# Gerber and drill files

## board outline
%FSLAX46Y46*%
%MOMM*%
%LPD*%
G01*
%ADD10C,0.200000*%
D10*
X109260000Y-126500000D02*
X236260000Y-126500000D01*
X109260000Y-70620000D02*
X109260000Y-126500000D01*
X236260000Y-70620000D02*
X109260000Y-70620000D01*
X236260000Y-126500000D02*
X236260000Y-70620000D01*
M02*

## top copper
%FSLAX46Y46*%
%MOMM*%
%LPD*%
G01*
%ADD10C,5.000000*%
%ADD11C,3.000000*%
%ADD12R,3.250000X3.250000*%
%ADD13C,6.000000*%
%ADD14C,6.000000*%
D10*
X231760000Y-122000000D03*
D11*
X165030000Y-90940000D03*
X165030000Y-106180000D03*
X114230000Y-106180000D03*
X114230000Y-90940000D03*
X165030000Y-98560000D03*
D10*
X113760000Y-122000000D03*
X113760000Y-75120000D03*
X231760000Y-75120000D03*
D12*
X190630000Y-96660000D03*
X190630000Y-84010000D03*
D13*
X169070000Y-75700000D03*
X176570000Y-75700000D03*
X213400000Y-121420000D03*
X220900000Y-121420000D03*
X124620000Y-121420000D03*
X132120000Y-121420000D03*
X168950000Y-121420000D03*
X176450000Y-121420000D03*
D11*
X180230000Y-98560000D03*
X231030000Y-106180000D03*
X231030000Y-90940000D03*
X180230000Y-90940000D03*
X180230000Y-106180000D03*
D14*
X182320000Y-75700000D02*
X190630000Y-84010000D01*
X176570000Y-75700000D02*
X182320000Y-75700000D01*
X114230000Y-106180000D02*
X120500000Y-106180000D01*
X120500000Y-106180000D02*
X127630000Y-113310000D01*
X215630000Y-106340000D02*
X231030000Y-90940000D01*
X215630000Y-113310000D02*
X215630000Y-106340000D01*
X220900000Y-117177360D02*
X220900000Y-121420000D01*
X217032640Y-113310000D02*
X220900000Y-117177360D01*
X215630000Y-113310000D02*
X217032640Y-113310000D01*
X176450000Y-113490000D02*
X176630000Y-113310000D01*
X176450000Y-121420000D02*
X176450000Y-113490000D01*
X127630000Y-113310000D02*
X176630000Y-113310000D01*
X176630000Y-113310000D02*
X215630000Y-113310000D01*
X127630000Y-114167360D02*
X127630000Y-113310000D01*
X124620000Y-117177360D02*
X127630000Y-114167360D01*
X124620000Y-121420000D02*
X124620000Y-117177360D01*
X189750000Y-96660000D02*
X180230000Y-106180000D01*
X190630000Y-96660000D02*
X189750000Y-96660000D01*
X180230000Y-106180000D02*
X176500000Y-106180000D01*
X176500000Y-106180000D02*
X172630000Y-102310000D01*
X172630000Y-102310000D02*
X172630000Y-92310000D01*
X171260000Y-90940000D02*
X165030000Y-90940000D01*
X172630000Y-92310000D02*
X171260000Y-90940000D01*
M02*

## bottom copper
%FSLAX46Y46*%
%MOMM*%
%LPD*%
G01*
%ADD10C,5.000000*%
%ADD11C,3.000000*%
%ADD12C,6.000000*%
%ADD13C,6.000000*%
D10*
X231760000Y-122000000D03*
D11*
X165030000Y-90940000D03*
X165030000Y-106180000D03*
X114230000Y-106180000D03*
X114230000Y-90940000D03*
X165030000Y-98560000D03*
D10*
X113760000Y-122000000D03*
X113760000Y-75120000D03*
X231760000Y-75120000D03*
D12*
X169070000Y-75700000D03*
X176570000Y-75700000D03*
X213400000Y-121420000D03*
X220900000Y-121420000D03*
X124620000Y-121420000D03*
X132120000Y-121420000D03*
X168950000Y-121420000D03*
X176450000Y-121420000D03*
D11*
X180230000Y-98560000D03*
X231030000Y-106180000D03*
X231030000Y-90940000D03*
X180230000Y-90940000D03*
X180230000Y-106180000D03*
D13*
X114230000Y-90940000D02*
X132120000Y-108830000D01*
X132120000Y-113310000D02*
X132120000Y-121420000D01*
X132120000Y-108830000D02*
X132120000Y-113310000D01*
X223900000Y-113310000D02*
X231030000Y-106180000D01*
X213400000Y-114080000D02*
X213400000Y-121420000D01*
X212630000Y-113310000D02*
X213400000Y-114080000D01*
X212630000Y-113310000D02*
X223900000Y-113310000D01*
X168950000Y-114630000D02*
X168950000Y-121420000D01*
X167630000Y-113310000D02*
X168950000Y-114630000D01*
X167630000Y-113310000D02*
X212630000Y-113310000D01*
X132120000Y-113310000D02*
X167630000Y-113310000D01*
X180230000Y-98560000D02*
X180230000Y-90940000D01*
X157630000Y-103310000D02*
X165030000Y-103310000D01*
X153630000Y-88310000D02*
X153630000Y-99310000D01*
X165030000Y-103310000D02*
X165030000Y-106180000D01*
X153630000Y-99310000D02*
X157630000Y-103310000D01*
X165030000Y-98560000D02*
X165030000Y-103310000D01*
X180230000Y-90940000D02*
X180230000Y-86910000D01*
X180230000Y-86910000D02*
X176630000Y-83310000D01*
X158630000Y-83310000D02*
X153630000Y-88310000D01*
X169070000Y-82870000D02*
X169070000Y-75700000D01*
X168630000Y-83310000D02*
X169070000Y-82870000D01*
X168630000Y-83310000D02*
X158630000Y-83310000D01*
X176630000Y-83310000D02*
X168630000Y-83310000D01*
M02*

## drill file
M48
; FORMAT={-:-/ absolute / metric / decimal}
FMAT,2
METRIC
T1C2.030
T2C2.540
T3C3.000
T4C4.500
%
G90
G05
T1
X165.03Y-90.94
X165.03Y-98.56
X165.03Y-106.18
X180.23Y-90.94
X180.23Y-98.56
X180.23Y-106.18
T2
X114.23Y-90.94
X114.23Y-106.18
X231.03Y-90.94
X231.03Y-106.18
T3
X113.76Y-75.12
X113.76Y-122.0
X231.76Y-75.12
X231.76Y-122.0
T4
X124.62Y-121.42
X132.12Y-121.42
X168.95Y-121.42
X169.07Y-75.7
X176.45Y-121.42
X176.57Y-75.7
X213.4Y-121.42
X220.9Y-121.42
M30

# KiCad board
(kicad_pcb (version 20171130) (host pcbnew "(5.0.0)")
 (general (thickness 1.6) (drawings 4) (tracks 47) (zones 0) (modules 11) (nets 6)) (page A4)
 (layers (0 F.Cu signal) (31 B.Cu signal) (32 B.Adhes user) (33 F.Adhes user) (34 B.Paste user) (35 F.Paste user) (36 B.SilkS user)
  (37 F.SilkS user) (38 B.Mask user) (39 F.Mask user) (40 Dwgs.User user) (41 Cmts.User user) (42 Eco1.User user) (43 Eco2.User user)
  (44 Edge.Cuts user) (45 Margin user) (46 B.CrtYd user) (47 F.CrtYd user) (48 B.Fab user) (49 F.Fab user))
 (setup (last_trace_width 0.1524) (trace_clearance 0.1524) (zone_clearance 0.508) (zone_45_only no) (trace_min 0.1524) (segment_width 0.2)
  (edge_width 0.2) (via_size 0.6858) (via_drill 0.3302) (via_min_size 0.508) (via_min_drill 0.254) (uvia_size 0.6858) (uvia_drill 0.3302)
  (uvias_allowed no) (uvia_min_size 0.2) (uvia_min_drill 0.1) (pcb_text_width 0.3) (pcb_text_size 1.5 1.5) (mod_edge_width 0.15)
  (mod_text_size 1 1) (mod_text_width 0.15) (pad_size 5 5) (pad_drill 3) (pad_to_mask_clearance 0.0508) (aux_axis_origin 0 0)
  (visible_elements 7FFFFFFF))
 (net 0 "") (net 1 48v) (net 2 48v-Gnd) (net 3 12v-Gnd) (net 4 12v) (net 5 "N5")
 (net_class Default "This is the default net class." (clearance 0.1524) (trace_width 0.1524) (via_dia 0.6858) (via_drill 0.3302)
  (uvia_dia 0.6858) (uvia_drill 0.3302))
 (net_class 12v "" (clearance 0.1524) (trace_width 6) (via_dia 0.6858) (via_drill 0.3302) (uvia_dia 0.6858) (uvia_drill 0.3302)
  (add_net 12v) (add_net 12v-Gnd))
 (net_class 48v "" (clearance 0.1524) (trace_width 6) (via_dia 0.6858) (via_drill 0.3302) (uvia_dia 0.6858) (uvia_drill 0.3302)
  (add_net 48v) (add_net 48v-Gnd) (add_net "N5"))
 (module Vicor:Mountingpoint (layer F.Cu) (at 252.73 96.52)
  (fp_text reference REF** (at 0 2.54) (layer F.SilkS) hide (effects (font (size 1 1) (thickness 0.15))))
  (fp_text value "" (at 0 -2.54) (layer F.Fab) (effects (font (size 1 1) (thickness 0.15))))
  (pad "" thru_hole circle (at -20.97 25.48) (size 5 5) (drill 3) (layers *.Cu *.Mask)))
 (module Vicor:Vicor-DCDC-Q (layer B.Cu) (at 139.63 98.56 180)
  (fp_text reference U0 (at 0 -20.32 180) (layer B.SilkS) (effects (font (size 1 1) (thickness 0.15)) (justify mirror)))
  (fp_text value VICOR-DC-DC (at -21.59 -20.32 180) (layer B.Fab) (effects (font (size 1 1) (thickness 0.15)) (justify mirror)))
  (pad 1 thru_hole circle (at -25.4 7.62 180) (size 3 3) (drill 2.03) (layers *.Cu *.Mask) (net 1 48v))
  (pad 3 thru_hole circle (at -25.4 -7.62 180) (size 3 3) (drill 2.03) (layers *.Cu *.Mask) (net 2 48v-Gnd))
  (pad 4 thru_hole circle (at 25.4 -7.62 180) (size 3 3) (drill 2.54) (layers *.Cu *.Mask) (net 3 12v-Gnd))
  (pad 5 thru_hole circle (at 25.4 7.62 180) (size 3 3) (drill 2.54) (layers *.Cu *.Mask) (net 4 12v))
  (pad 2 thru_hole circle (at -25.4 0 180) (size 3 3) (drill 2.03) (layers *.Cu *.Mask) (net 2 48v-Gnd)))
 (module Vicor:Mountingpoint (layer F.Cu) (at 263.47 99.06)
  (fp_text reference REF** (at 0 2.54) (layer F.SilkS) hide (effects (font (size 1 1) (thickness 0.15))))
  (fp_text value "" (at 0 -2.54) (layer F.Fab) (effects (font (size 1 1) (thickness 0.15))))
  (pad "" thru_hole circle (at -149.71 22.94) (size 5 5) (drill 3) (layers *.Cu *.Mask)))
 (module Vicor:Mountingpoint (layer F.Cu) (at 255.27 81.28)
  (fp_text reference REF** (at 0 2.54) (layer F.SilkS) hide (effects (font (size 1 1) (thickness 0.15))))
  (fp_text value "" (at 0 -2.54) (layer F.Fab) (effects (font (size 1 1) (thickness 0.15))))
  (pad "" thru_hole circle (at -141.51 -6.16) (size 5 5) (drill 3) (layers *.Cu *.Mask)))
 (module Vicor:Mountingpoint (layer F.Cu) (at 243.42 75.58)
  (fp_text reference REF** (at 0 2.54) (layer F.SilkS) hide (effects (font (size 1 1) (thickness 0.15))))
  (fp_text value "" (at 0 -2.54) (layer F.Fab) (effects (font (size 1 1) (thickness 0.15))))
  (pad "" thru_hole circle (at -11.66 -0.46) (size 5 5) (drill 3) (layers *.Cu *.Mask)))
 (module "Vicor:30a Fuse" (layer F.Cu) (at 190.63 90.31 270)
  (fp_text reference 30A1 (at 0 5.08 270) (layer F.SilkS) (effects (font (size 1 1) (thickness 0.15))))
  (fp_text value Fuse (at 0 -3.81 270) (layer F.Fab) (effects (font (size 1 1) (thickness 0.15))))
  (pad 2 smd rect (at 6.35 0 270) (size 3.25 3.25) (layers F.Cu F.Paste F.Mask) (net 1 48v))
  (pad 1 smd rect (at -6.3 0 270) (size 3.25 3.25) (layers F.Cu F.Paste F.Mask) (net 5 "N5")))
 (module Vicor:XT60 (layer F.Cu) (at 176.57 75.7 180)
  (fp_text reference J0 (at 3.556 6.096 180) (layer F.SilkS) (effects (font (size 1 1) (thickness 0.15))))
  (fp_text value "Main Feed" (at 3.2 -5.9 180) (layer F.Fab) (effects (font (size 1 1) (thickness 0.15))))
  (pad 2 thru_hole circle (at 7.5 0 180) (size 6 6) (drill 4.5) (layers *.Cu *.Mask F.SilkS) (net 2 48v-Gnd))
  (pad 1 thru_hole circle (at 0 0 180) (size 6 6) (drill 4.5) (layers *.Cu *.Mask F.SilkS) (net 5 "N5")))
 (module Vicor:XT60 (layer F.Cu) (at 213.4 121.42)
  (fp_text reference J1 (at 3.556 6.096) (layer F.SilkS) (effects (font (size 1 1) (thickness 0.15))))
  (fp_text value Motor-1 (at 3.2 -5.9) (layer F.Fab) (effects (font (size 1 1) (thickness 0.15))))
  (pad 1 thru_hole circle (at 0 0) (size 6 6) (drill 4.5) (layers *.Cu *.Mask F.SilkS) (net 4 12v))
  (pad 2 thru_hole circle (at 7.5 0) (size 6 6) (drill 4.5) (layers *.Cu *.Mask F.SilkS) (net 3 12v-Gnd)))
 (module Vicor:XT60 (layer F.Cu) (at 132.12 121.42 180)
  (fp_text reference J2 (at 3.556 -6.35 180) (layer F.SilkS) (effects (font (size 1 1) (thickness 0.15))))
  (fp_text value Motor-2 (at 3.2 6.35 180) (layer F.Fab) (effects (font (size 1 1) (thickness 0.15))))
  (pad 2 thru_hole circle (at 7.5 0 180) (size 6 6) (drill 4.5) (layers *.Cu *.Mask F.SilkS) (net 3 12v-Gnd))
  (pad 1 thru_hole circle (at 0 0 180) (size 6 6) (drill 4.5) (layers *.Cu *.Mask F.SilkS) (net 4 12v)))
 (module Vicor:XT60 (layer F.Cu) (at 168.95 121.42)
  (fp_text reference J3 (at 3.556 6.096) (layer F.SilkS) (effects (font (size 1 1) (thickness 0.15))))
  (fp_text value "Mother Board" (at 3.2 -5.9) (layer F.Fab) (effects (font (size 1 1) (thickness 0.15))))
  (pad 1 thru_hole circle (at 0 0) (size 6 6) (drill 4.5) (layers *.Cu *.Mask F.SilkS) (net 4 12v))
  (pad 2 thru_hole circle (at 7.5 0) (size 6 6) (drill 4.5) (layers *.Cu *.Mask F.SilkS) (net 3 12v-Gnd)))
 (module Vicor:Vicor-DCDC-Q (layer B.Cu) (at 205.63 98.56)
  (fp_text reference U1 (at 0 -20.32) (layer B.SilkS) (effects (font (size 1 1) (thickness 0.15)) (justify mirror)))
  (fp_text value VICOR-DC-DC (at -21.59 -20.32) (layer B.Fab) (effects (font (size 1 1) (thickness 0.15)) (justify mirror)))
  (pad 2 thru_hole circle (at -25.4 0) (size 3 3) (drill 2.03) (layers *.Cu *.Mask) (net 2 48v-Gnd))
  (pad 5 thru_hole circle (at 25.4 7.62) (size 3 3) (drill 2.54) (layers *.Cu *.Mask) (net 4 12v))
  (pad 4 thru_hole circle (at 25.4 -7.62) (size 3 3) (drill 2.54) (layers *.Cu *.Mask) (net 3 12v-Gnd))
  (pad 3 thru_hole circle (at -25.4 -7.62) (size 3 3) (drill 2.03) (layers *.Cu *.Mask) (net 2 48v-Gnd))
  (pad 1 thru_hole circle (at -25.4 7.62) (size 3 3) (drill 2.03) (layers *.Cu *.Mask) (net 1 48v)))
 (gr_line (start 109.26 126.5) (end 236.26 126.5) (layer Edge.Cuts) (width 0.2))
 (gr_line (start 109.26 70.62) (end 109.26 126.5) (layer Edge.Cuts) (width 0.2))
 (gr_line (start 236.26 70.62) (end 109.26 70.62) (layer Edge.Cuts) (width 0.2))
 (gr_line (start 236.26 126.5) (end 236.26 70.62) (layer Edge.Cuts) (width 0.2))
 (segment (start 182.32 75.7) (end 190.63 84.01) (width 6) (layer F.Cu) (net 5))
 (segment (start 176.57 75.7) (end 182.32 75.7) (width 6) (layer F.Cu) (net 5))
 (segment (start 114.23 90.94) (end 132.12 108.83) (width 6) (layer B.Cu) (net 4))
 (segment (start 132.12 113.31) (end 132.12 121.42) (width 6) (layer B.Cu) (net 4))
 (segment (start 132.12 108.83) (end 132.12 113.31) (width 6) (layer B.Cu) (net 4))
 (segment (start 223.9 113.31) (end 231.03 106.18) (width 6) (layer B.Cu) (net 4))
 (segment (start 213.4 114.08) (end 213.4 121.42) (width 6) (layer B.Cu) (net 4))
 (segment (start 212.63 113.31) (end 213.4 114.08) (width 6) (layer B.Cu) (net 4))
 (segment (start 212.63 113.31) (end 223.9 113.31) (width 6) (layer B.Cu) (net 4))
 (segment (start 168.95 114.63) (end 168.95 121.42) (width 6) (layer B.Cu) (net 4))
 (segment (start 167.63 113.31) (end 168.95 114.63) (width 6) (layer B.Cu) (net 4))
 (segment (start 167.63 113.31) (end 212.63 113.31) (width 6) (layer B.Cu) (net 4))
 (segment (start 132.12 113.31) (end 167.63 113.31) (width 6) (layer B.Cu) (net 4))
 (segment (start 114.23 106.18) (end 120.5 106.18) (width 6) (layer F.Cu) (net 3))
 (segment (start 120.5 106.18) (end 127.63 113.31) (width 6) (layer F.Cu) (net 3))
 (segment (start 215.63 106.34) (end 231.03 90.94) (width 6) (layer F.Cu) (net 3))
 (segment (start 215.63 113.31) (end 215.63 106.34) (width 6) (layer F.Cu) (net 3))
 (segment (start 220.9 117.17736) (end 220.9 121.42) (width 6) (layer F.Cu) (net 3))
 (segment (start 217.03264 113.31) (end 220.9 117.17736) (width 6) (layer F.Cu) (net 3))
 (segment (start 215.63 113.31) (end 217.03264 113.31) (width 6) (layer F.Cu) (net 3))
 (segment (start 176.45 113.49) (end 176.63 113.31) (width 6) (layer F.Cu) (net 3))
 (segment (start 176.45 121.42) (end 176.45 113.49) (width 6) (layer F.Cu) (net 3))
 (segment (start 127.63 113.31) (end 176.63 113.31) (width 6) (layer F.Cu) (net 3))
 (segment (start 176.63 113.31) (end 215.63 113.31) (width 6) (layer F.Cu) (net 3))
 (segment (start 127.63 114.16736) (end 127.63 113.31) (width 6) (layer F.Cu) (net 3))
 (segment (start 124.62 117.17736) (end 127.63 114.16736) (width 6) (layer F.Cu) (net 3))
 (segment (start 124.62 121.42) (end 124.62 117.17736) (width 6) (layer F.Cu) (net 3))
 (segment (start 189.75 96.66) (end 180.23 106.18) (width 6) (layer F.Cu) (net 1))
 (segment (start 190.63 96.66) (end 189.75 96.66) (width 6) (layer F.Cu) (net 1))
 (segment (start 180.23 106.18) (end 176.5 106.18) (width 6) (layer F.Cu) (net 1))
 (segment (start 176.5 106.18) (end 172.63 102.31) (width 6) (layer F.Cu) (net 1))
 (segment (start 172.63 102.31) (end 172.63 92.31) (width 6) (layer F.Cu) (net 1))
 (segment (start 171.26 90.94) (end 165.03 90.94) (width 6) (layer F.Cu) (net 1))
 (segment (start 172.63 92.31) (end 171.26 90.94) (width 6) (layer F.Cu) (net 1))
 (segment (start 180.23 98.56) (end 180.23 90.94) (width 6) (layer B.Cu) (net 2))
 (segment (start 157.63 103.31) (end 165.03 103.31) (width 6) (layer B.Cu) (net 2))
 (segment (start 153.63 88.31) (end 153.63 99.31) (width 6) (layer B.Cu) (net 2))
 (segment (start 165.03 103.31) (end 165.03 106.18) (width 6) (layer B.Cu) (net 2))
 (segment (start 153.63 99.31) (end 157.63 103.31) (width 6) (layer B.Cu) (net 2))
 (segment (start 165.03 98.56) (end 165.03 103.31) (width 6) (layer B.Cu) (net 2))
 (segment (start 180.23 90.94) (end 180.23 86.91) (width 6) (layer B.Cu) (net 2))
 (segment (start 180.23 86.91) (end 176.63 83.31) (width 6) (layer B.Cu) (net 2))
 (segment (start 158.63 83.31) (end 153.63 88.31) (width 6) (layer B.Cu) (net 2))
 (segment (start 169.07 82.87) (end 169.07 75.7) (width 6) (layer B.Cu) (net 2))
 (segment (start 168.63 83.31) (end 169.07 82.87) (width 6) (layer B.Cu) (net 2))
 (segment (start 168.63 83.31) (end 158.63 83.31) (width 6) (layer B.Cu) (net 2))
 (segment (start 176.63 83.31) (end 168.63 83.31) (width 6) (layer B.Cu) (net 2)))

